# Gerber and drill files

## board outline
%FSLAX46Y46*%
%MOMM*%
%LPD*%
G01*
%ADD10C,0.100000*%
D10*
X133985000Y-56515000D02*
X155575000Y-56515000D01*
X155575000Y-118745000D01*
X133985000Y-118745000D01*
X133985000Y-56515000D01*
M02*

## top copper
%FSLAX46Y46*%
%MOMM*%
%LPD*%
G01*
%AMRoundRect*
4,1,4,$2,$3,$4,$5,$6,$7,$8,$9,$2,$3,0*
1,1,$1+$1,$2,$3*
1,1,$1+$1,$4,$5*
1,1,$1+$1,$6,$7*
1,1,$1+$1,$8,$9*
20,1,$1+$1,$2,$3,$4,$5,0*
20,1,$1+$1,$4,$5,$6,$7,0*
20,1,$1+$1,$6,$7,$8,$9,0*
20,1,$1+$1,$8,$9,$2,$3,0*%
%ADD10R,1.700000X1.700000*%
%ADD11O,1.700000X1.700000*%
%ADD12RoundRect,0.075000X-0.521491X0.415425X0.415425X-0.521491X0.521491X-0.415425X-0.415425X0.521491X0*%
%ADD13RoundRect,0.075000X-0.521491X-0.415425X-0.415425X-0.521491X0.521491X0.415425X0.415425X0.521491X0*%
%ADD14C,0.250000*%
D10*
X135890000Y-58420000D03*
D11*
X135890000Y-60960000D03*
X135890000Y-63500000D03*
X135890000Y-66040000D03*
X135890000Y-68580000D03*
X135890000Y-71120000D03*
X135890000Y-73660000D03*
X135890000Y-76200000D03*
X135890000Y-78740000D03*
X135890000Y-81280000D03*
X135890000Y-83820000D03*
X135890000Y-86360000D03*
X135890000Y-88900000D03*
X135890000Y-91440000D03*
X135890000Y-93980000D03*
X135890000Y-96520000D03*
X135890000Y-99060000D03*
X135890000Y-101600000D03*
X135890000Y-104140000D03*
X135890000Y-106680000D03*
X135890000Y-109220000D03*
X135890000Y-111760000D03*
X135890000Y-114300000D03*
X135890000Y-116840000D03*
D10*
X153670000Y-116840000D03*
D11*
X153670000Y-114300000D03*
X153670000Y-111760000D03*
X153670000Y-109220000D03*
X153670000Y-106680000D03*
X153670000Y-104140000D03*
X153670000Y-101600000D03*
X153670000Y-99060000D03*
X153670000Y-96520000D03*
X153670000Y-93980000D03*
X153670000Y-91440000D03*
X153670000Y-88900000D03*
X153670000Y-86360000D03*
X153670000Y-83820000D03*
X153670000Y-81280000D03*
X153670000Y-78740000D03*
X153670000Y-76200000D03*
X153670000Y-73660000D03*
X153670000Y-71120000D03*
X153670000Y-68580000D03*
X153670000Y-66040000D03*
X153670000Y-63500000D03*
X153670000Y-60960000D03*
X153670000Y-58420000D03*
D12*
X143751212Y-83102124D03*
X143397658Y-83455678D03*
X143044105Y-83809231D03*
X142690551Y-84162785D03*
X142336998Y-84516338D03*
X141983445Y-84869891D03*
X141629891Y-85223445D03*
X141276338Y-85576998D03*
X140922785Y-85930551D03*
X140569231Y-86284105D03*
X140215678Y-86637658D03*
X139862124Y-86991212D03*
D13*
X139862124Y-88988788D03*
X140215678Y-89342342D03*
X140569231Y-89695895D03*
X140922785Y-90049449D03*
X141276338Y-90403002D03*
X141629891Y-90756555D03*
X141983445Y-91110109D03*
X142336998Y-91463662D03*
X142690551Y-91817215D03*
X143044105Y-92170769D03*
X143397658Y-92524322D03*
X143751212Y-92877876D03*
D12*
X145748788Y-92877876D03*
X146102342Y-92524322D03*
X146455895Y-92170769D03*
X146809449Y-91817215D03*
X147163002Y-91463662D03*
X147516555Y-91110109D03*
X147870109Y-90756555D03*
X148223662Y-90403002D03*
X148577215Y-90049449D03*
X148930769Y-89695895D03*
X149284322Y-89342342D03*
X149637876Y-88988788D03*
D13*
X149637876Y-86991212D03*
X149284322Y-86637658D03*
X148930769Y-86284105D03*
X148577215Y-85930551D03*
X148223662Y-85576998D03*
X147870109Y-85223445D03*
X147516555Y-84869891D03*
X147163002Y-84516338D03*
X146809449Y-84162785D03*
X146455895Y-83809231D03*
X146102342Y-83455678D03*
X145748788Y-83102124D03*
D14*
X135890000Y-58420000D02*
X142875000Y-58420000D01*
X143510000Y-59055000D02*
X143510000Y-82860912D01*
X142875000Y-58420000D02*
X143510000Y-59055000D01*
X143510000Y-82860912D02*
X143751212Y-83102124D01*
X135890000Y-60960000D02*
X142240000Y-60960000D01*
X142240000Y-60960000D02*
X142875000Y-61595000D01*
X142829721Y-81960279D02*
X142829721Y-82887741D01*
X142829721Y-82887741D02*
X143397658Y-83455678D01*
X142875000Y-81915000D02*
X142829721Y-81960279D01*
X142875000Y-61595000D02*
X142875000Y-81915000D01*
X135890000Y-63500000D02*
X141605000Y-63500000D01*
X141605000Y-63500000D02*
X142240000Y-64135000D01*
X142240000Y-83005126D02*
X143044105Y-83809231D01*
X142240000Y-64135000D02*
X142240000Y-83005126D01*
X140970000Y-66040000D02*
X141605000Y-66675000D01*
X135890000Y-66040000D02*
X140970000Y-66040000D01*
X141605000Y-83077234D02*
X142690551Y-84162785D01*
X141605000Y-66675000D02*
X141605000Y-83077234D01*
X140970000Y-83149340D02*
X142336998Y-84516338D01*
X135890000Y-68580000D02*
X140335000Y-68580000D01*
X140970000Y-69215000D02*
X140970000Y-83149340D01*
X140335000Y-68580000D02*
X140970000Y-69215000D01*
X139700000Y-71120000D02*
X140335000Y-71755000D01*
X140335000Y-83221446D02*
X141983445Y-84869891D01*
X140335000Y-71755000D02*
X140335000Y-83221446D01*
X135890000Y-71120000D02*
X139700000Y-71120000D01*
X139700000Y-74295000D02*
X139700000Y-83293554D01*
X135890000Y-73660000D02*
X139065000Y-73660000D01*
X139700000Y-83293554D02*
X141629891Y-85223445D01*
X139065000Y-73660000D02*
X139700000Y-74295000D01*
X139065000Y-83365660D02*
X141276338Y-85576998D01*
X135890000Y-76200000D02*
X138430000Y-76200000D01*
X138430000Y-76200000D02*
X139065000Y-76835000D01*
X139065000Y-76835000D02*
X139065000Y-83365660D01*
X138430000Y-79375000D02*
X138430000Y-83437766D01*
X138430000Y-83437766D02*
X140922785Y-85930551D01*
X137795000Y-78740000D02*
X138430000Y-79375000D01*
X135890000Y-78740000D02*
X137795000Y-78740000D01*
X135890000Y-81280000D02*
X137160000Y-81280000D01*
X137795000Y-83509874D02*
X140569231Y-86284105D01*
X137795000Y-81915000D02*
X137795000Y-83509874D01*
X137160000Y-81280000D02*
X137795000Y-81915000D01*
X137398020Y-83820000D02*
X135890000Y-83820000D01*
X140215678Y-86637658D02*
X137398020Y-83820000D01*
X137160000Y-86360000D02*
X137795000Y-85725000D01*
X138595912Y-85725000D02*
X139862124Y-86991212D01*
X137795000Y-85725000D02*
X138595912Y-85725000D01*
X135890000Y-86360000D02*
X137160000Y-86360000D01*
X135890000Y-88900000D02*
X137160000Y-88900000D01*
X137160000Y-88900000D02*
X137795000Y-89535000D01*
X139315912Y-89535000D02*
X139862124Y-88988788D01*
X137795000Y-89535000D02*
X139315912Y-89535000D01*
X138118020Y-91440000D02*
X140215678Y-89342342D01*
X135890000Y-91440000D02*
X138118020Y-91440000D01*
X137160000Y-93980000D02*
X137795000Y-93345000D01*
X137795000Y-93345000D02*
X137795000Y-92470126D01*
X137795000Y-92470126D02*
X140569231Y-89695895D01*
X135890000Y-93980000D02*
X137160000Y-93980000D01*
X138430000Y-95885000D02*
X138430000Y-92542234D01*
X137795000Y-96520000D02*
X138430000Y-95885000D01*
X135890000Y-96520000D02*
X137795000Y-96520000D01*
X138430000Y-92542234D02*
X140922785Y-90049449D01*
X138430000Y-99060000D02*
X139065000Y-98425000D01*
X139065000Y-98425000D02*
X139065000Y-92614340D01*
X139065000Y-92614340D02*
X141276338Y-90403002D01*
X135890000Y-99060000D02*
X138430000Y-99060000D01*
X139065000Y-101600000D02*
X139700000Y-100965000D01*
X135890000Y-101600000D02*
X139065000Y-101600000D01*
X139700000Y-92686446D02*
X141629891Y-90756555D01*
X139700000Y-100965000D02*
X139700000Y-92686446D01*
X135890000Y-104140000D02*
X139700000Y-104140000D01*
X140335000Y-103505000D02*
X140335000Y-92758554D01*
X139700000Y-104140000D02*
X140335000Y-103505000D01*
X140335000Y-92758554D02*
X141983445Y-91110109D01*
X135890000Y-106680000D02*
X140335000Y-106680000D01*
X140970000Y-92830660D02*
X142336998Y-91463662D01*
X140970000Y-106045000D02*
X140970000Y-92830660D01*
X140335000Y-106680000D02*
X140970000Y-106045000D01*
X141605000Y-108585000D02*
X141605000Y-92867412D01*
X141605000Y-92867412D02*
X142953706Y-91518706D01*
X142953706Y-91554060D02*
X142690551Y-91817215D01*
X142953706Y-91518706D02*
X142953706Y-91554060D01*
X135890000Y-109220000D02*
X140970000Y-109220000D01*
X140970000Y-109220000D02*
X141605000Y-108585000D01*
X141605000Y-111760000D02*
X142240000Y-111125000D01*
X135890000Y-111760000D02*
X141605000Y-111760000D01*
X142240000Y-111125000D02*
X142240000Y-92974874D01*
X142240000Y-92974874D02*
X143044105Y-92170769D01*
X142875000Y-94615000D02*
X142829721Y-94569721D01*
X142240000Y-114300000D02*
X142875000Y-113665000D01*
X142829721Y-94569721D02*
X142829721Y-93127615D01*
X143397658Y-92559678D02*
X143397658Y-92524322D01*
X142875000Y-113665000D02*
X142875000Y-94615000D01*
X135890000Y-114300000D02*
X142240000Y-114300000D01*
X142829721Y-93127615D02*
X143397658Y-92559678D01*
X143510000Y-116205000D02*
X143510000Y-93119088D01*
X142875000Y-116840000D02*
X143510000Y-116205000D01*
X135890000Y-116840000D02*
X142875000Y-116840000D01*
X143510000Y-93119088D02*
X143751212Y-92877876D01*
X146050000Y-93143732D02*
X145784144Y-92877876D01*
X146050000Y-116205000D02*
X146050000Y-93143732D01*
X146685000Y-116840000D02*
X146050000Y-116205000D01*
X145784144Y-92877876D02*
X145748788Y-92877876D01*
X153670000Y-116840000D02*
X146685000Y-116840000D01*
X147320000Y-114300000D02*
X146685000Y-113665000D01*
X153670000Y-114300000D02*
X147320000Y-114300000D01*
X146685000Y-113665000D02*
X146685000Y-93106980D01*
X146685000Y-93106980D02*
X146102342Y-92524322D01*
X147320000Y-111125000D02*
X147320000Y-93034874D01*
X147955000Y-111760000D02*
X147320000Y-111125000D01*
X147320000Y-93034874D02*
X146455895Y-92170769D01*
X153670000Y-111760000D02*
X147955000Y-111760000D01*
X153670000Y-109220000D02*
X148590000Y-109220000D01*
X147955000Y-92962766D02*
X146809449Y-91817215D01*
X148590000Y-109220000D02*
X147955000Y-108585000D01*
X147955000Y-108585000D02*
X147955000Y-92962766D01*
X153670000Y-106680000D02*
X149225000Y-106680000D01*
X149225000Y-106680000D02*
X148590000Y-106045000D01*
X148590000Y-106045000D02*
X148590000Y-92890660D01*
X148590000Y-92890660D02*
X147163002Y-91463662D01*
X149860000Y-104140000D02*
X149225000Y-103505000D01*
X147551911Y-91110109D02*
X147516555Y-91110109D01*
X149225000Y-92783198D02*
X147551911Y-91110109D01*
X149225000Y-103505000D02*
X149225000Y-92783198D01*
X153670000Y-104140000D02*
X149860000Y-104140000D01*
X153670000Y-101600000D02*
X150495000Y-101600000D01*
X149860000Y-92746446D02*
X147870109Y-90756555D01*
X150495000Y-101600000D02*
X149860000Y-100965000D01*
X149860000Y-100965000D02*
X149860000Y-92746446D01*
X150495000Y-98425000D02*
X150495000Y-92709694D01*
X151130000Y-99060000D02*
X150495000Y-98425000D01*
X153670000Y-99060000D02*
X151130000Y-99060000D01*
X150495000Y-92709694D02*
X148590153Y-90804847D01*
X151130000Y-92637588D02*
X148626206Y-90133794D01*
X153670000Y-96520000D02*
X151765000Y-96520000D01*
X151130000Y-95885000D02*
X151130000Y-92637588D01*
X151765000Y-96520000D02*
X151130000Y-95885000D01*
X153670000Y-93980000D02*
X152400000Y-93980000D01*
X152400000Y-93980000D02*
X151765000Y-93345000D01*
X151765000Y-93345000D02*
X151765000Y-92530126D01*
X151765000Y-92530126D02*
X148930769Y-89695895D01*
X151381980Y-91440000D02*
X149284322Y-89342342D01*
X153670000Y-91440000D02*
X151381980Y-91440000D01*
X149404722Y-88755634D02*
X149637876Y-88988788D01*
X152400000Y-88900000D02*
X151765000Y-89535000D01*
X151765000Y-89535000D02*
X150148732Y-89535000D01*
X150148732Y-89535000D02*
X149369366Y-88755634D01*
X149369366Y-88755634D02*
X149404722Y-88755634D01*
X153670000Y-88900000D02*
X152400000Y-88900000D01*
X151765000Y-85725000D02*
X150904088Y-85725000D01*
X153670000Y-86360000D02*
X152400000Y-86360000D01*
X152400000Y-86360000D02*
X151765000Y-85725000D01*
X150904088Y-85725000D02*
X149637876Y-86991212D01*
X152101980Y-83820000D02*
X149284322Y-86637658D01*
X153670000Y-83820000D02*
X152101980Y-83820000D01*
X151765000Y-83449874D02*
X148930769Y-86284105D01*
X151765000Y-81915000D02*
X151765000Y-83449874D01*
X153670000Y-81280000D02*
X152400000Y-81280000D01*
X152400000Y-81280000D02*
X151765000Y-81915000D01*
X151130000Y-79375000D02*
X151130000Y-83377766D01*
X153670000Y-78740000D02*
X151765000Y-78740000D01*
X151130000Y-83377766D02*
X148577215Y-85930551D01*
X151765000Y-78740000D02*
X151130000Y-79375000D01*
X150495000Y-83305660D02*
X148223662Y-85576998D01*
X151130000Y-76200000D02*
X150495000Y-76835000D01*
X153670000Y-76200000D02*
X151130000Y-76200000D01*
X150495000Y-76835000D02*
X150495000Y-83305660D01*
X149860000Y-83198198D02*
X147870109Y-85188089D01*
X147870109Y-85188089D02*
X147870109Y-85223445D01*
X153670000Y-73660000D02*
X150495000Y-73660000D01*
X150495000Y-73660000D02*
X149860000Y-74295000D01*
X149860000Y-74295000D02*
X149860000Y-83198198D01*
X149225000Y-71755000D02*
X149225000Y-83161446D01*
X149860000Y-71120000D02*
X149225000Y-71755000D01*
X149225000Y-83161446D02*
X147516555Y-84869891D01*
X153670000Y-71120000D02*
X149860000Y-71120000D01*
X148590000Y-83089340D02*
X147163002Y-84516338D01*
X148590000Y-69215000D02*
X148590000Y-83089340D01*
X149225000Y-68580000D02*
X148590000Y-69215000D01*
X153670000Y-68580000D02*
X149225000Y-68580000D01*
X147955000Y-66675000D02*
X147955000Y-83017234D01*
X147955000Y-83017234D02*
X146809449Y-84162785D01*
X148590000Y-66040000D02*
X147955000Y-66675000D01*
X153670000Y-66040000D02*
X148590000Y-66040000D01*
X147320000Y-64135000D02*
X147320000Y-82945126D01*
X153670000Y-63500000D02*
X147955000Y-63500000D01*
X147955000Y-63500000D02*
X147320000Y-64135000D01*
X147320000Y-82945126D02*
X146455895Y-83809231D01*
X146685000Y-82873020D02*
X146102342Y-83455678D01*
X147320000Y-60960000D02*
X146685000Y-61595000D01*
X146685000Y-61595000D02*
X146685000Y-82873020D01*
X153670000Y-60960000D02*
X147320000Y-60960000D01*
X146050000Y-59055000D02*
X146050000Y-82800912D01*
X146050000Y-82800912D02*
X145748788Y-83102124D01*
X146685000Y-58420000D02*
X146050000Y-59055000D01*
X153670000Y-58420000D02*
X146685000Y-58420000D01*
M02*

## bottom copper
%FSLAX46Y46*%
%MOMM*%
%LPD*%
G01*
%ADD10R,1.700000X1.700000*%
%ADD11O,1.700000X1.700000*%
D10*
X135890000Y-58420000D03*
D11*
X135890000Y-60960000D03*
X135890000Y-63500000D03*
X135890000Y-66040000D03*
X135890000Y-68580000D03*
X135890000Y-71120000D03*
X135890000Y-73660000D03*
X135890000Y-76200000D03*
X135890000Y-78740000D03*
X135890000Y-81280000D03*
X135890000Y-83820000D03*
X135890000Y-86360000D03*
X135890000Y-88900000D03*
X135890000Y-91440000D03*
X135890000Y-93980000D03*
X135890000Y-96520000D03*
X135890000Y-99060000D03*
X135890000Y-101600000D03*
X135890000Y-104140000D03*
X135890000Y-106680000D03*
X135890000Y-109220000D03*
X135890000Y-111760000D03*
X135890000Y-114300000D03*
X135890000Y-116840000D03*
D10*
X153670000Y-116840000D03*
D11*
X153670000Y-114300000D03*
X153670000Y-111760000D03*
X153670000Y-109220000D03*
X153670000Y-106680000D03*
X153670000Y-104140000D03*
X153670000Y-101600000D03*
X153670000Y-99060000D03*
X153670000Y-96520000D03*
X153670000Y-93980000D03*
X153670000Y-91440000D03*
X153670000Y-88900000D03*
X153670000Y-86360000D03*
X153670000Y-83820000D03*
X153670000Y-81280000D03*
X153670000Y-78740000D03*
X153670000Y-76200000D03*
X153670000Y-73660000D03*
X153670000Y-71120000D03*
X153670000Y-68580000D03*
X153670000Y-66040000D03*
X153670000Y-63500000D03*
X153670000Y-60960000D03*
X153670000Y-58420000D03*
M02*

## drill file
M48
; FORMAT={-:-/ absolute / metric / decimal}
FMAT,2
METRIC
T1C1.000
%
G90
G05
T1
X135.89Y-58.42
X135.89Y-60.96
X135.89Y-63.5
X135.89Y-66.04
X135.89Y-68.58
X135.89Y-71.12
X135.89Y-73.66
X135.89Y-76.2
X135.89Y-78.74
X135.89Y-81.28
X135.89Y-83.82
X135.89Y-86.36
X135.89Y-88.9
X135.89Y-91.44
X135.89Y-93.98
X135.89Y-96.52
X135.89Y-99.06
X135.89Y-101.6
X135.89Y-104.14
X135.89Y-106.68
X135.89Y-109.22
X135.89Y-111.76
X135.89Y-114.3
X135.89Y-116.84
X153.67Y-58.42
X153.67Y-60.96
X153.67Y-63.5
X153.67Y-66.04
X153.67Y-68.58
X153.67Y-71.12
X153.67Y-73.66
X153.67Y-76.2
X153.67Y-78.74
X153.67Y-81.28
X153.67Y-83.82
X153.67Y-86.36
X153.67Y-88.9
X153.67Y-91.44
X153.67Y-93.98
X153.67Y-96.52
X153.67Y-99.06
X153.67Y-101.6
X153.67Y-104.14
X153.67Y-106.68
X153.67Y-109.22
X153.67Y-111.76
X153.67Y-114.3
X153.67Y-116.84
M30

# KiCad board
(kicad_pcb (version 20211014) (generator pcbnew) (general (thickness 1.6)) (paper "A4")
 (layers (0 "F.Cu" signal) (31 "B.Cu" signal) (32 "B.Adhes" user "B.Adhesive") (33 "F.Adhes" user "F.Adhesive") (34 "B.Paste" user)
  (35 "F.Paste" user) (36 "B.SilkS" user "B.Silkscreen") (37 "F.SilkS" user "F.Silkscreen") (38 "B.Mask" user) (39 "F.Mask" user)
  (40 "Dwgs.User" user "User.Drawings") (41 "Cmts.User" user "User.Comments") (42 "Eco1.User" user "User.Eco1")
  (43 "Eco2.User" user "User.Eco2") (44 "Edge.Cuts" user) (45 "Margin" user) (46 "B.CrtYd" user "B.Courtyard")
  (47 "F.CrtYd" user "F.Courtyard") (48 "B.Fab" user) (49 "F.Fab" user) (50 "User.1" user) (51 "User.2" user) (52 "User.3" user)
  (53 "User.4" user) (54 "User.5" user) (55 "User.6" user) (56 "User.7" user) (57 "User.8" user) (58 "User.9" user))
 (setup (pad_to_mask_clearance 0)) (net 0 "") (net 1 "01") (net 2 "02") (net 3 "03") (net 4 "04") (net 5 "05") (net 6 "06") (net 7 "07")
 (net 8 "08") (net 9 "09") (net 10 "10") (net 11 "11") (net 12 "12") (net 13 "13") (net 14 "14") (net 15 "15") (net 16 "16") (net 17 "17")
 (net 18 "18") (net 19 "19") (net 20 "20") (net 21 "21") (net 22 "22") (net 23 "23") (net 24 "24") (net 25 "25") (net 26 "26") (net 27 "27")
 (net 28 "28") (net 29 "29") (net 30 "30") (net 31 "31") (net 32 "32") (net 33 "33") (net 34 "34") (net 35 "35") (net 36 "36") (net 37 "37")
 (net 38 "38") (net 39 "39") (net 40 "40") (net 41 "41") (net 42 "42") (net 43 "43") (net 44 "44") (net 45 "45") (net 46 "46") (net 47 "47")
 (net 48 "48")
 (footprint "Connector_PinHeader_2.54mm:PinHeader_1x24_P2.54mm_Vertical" (layer "F.Cu") (at 135.89 58.42)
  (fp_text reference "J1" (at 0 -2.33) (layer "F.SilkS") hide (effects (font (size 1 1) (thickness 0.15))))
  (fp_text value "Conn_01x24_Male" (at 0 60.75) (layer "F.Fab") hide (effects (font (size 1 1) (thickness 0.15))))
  (pad "1" thru_hole rect (at 0 0) (size 1.7 1.7) (drill 1) (layers *.Cu *.Mask) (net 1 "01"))
  (pad "2" thru_hole oval (at 0 2.54) (size 1.7 1.7) (drill 1) (layers *.Cu *.Mask) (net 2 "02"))
  (pad "3" thru_hole oval (at 0 5.08) (size 1.7 1.7) (drill 1) (layers *.Cu *.Mask) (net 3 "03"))
  (pad "4" thru_hole oval (at 0 7.62) (size 1.7 1.7) (drill 1) (layers *.Cu *.Mask) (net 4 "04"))
  (pad "5" thru_hole oval (at 0 10.16) (size 1.7 1.7) (drill 1) (layers *.Cu *.Mask) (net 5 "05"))
  (pad "6" thru_hole oval (at 0 12.7) (size 1.7 1.7) (drill 1) (layers *.Cu *.Mask) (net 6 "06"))
  (pad "7" thru_hole oval (at 0 15.24) (size 1.7 1.7) (drill 1) (layers *.Cu *.Mask) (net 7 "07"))
  (pad "8" thru_hole oval (at 0 17.78) (size 1.7 1.7) (drill 1) (layers *.Cu *.Mask) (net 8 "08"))
  (pad "9" thru_hole oval (at 0 20.32) (size 1.7 1.7) (drill 1) (layers *.Cu *.Mask) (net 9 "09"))
  (pad "10" thru_hole oval (at 0 22.86) (size 1.7 1.7) (drill 1) (layers *.Cu *.Mask) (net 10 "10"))
  (pad "11" thru_hole oval (at 0 25.4) (size 1.7 1.7) (drill 1) (layers *.Cu *.Mask) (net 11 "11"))
  (pad "12" thru_hole oval (at 0 27.94) (size 1.7 1.7) (drill 1) (layers *.Cu *.Mask) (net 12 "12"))
  (pad "13" thru_hole oval (at 0 30.48) (size 1.7 1.7) (drill 1) (layers *.Cu *.Mask) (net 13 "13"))
  (pad "14" thru_hole oval (at 0 33.02) (size 1.7 1.7) (drill 1) (layers *.Cu *.Mask) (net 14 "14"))
  (pad "15" thru_hole oval (at 0 35.56) (size 1.7 1.7) (drill 1) (layers *.Cu *.Mask) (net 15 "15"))
  (pad "16" thru_hole oval (at 0 38.1) (size 1.7 1.7) (drill 1) (layers *.Cu *.Mask) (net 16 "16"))
  (pad "17" thru_hole oval (at 0 40.64) (size 1.7 1.7) (drill 1) (layers *.Cu *.Mask) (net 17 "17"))
  (pad "18" thru_hole oval (at 0 43.18) (size 1.7 1.7) (drill 1) (layers *.Cu *.Mask) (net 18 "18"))
  (pad "19" thru_hole oval (at 0 45.72) (size 1.7 1.7) (drill 1) (layers *.Cu *.Mask) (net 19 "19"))
  (pad "20" thru_hole oval (at 0 48.26) (size 1.7 1.7) (drill 1) (layers *.Cu *.Mask) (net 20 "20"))
  (pad "21" thru_hole oval (at 0 50.8) (size 1.7 1.7) (drill 1) (layers *.Cu *.Mask) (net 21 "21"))
  (pad "22" thru_hole oval (at 0 53.34) (size 1.7 1.7) (drill 1) (layers *.Cu *.Mask) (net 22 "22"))
  (pad "23" thru_hole oval (at 0 55.88) (size 1.7 1.7) (drill 1) (layers *.Cu *.Mask) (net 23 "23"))
  (pad "24" thru_hole oval (at 0 58.42) (size 1.7 1.7) (drill 1) (layers *.Cu *.Mask) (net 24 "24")))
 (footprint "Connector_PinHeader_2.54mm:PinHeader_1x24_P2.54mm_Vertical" (layer "F.Cu") (at 153.67 116.84 180)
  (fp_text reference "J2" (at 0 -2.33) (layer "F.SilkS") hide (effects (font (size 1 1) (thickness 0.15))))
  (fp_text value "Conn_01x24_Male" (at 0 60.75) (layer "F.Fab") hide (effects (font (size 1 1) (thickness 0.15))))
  (pad "1" thru_hole rect (at 0 0 180) (size 1.7 1.7) (drill 1) (layers *.Cu *.Mask) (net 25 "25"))
  (pad "2" thru_hole oval (at 0 2.54 180) (size 1.7 1.7) (drill 1) (layers *.Cu *.Mask) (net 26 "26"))
  (pad "3" thru_hole oval (at 0 5.08 180) (size 1.7 1.7) (drill 1) (layers *.Cu *.Mask) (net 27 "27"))
  (pad "4" thru_hole oval (at 0 7.62 180) (size 1.7 1.7) (drill 1) (layers *.Cu *.Mask) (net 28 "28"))
  (pad "5" thru_hole oval (at 0 10.16 180) (size 1.7 1.7) (drill 1) (layers *.Cu *.Mask) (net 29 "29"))
  (pad "6" thru_hole oval (at 0 12.7 180) (size 1.7 1.7) (drill 1) (layers *.Cu *.Mask) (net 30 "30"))
  (pad "7" thru_hole oval (at 0 15.24 180) (size 1.7 1.7) (drill 1) (layers *.Cu *.Mask) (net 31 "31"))
  (pad "8" thru_hole oval (at 0 17.78 180) (size 1.7 1.7) (drill 1) (layers *.Cu *.Mask) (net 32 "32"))
  (pad "9" thru_hole oval (at 0 20.32 180) (size 1.7 1.7) (drill 1) (layers *.Cu *.Mask) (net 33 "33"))
  (pad "10" thru_hole oval (at 0 22.86 180) (size 1.7 1.7) (drill 1) (layers *.Cu *.Mask) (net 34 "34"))
  (pad "11" thru_hole oval (at 0 25.4 180) (size 1.7 1.7) (drill 1) (layers *.Cu *.Mask) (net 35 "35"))
  (pad "12" thru_hole oval (at 0 27.94 180) (size 1.7 1.7) (drill 1) (layers *.Cu *.Mask) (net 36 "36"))
  (pad "13" thru_hole oval (at 0 30.48 180) (size 1.7 1.7) (drill 1) (layers *.Cu *.Mask) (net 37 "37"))
  (pad "14" thru_hole oval (at 0 33.02 180) (size 1.7 1.7) (drill 1) (layers *.Cu *.Mask) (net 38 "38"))
  (pad "15" thru_hole oval (at 0 35.56 180) (size 1.7 1.7) (drill 1) (layers *.Cu *.Mask) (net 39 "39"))
  (pad "16" thru_hole oval (at 0 38.1 180) (size 1.7 1.7) (drill 1) (layers *.Cu *.Mask) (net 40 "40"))
  (pad "17" thru_hole oval (at 0 40.64 180) (size 1.7 1.7) (drill 1) (layers *.Cu *.Mask) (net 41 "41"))
  (pad "18" thru_hole oval (at 0 43.18 180) (size 1.7 1.7) (drill 1) (layers *.Cu *.Mask) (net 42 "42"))
  (pad "19" thru_hole oval (at 0 45.72 180) (size 1.7 1.7) (drill 1) (layers *.Cu *.Mask) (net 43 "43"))
  (pad "20" thru_hole oval (at 0 48.26 180) (size 1.7 1.7) (drill 1) (layers *.Cu *.Mask) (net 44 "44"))
  (pad "21" thru_hole oval (at 0 50.8 180) (size 1.7 1.7) (drill 1) (layers *.Cu *.Mask) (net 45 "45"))
  (pad "22" thru_hole oval (at 0 53.34 180) (size 1.7 1.7) (drill 1) (layers *.Cu *.Mask) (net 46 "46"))
  (pad "23" thru_hole oval (at 0 55.88 180) (size 1.7 1.7) (drill 1) (layers *.Cu *.Mask) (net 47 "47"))
  (pad "24" thru_hole oval (at 0 58.42 180) (size 1.7 1.7) (drill 1) (layers *.Cu *.Mask) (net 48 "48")))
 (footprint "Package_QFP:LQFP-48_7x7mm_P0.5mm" (layer "F.Cu") (at 144.75 87.99 -45)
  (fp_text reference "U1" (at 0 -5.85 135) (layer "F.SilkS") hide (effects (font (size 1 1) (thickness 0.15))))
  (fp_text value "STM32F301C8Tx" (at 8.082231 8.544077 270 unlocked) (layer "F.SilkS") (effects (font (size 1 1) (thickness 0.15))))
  (pad "1" smd roundrect (at -4.1625 -2.75 315) (size 1.475 0.3) (layers "F.Cu" "F.Paste" "F.Mask") (roundrect_rratio 0.25) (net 1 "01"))
  (pad "2" smd roundrect (at -4.1625 -2.25 315) (size 1.475 0.3) (layers "F.Cu" "F.Paste" "F.Mask") (roundrect_rratio 0.25) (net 2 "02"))
  (pad "3" smd roundrect (at -4.1625 -1.75 315) (size 1.475 0.3) (layers "F.Cu" "F.Paste" "F.Mask") (roundrect_rratio 0.25) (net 3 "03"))
  (pad "4" smd roundrect (at -4.1625 -1.25 315) (size 1.475 0.3) (layers "F.Cu" "F.Paste" "F.Mask") (roundrect_rratio 0.25) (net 4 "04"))
  (pad "5" smd roundrect (at -4.1625 -0.75 315) (size 1.475 0.3) (layers "F.Cu" "F.Paste" "F.Mask") (roundrect_rratio 0.25) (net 5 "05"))
  (pad "6" smd roundrect (at -4.1625 -0.25 315) (size 1.475 0.3) (layers "F.Cu" "F.Paste" "F.Mask") (roundrect_rratio 0.25) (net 6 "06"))
  (pad "7" smd roundrect (at -4.1625 0.25 315) (size 1.475 0.3) (layers "F.Cu" "F.Paste" "F.Mask") (roundrect_rratio 0.25) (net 7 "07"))
  (pad "8" smd roundrect (at -4.1625 0.75 315) (size 1.475 0.3) (layers "F.Cu" "F.Paste" "F.Mask") (roundrect_rratio 0.25) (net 8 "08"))
  (pad "9" smd roundrect (at -4.1625 1.25 315) (size 1.475 0.3) (layers "F.Cu" "F.Paste" "F.Mask") (roundrect_rratio 0.25) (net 9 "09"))
  (pad "10" smd roundrect (at -4.1625 1.75 315) (size 1.475 0.3) (layers "F.Cu" "F.Paste" "F.Mask") (roundrect_rratio 0.25) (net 10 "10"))
  (pad "11" smd roundrect (at -4.1625 2.25 315) (size 1.475 0.3) (layers "F.Cu" "F.Paste" "F.Mask") (roundrect_rratio 0.25) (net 11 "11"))
  (pad "12" smd roundrect (at -4.1625 2.75 315) (size 1.475 0.3) (layers "F.Cu" "F.Paste" "F.Mask") (roundrect_rratio 0.25) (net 12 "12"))
  (pad "13" smd roundrect (at -2.75 4.1625 315) (size 0.3 1.475) (layers "F.Cu" "F.Paste" "F.Mask") (roundrect_rratio 0.25) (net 13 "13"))
  (pad "14" smd roundrect (at -2.25 4.1625 315) (size 0.3 1.475) (layers "F.Cu" "F.Paste" "F.Mask") (roundrect_rratio 0.25) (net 14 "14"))
  (pad "15" smd roundrect (at -1.75 4.1625 315) (size 0.3 1.475) (layers "F.Cu" "F.Paste" "F.Mask") (roundrect_rratio 0.25) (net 15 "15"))
  (pad "16" smd roundrect (at -1.25 4.1625 315) (size 0.3 1.475) (layers "F.Cu" "F.Paste" "F.Mask") (roundrect_rratio 0.25) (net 16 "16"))
  (pad "17" smd roundrect (at -0.75 4.1625 315) (size 0.3 1.475) (layers "F.Cu" "F.Paste" "F.Mask") (roundrect_rratio 0.25) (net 17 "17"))
  (pad "18" smd roundrect (at -0.25 4.1625 315) (size 0.3 1.475) (layers "F.Cu" "F.Paste" "F.Mask") (roundrect_rratio 0.25) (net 18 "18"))
  (pad "19" smd roundrect (at 0.25 4.1625 315) (size 0.3 1.475) (layers "F.Cu" "F.Paste" "F.Mask") (roundrect_rratio 0.25) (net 19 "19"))
  (pad "20" smd roundrect (at 0.75 4.1625 315) (size 0.3 1.475) (layers "F.Cu" "F.Paste" "F.Mask") (roundrect_rratio 0.25) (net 20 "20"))
  (pad "21" smd roundrect (at 1.25 4.1625 315) (size 0.3 1.475) (layers "F.Cu" "F.Paste" "F.Mask") (roundrect_rratio 0.25) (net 21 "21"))
  (pad "22" smd roundrect (at 1.75 4.1625 315) (size 0.3 1.475) (layers "F.Cu" "F.Paste" "F.Mask") (roundrect_rratio 0.25) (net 22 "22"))
  (pad "23" smd roundrect (at 2.25 4.1625 315) (size 0.3 1.475) (layers "F.Cu" "F.Paste" "F.Mask") (roundrect_rratio 0.25) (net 23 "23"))
  (pad "24" smd roundrect (at 2.75 4.1625 315) (size 0.3 1.475) (layers "F.Cu" "F.Paste" "F.Mask") (roundrect_rratio 0.25) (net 24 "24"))
  (pad "25" smd roundrect (at 4.1625 2.75 315) (size 1.475 0.3) (layers "F.Cu" "F.Paste" "F.Mask") (roundrect_rratio 0.25) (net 25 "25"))
  (pad "26" smd roundrect (at 4.1625 2.25 315) (size 1.475 0.3) (layers "F.Cu" "F.Paste" "F.Mask") (roundrect_rratio 0.25) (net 26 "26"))
  (pad "27" smd roundrect (at 4.1625 1.75 315) (size 1.475 0.3) (layers "F.Cu" "F.Paste" "F.Mask") (roundrect_rratio 0.25) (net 27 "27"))
  (pad "28" smd roundrect (at 4.1625 1.25 315) (size 1.475 0.3) (layers "F.Cu" "F.Paste" "F.Mask") (roundrect_rratio 0.25) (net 28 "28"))
  (pad "29" smd roundrect (at 4.1625 0.75 315) (size 1.475 0.3) (layers "F.Cu" "F.Paste" "F.Mask") (roundrect_rratio 0.25) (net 29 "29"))
  (pad "30" smd roundrect (at 4.1625 0.25 315) (size 1.475 0.3) (layers "F.Cu" "F.Paste" "F.Mask") (roundrect_rratio 0.25) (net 30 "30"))
  (pad "31" smd roundrect (at 4.1625 -0.25 315) (size 1.475 0.3) (layers "F.Cu" "F.Paste" "F.Mask") (roundrect_rratio 0.25) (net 31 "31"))
  (pad "32" smd roundrect (at 4.1625 -0.75 315) (size 1.475 0.3) (layers "F.Cu" "F.Paste" "F.Mask") (roundrect_rratio 0.25) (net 32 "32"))
  (pad "33" smd roundrect (at 4.1625 -1.25 315) (size 1.475 0.3) (layers "F.Cu" "F.Paste" "F.Mask") (roundrect_rratio 0.25) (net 33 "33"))
  (pad "34" smd roundrect (at 4.1625 -1.75 315) (size 1.475 0.3) (layers "F.Cu" "F.Paste" "F.Mask") (roundrect_rratio 0.25) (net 34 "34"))
  (pad "35" smd roundrect (at 4.1625 -2.25 315) (size 1.475 0.3) (layers "F.Cu" "F.Paste" "F.Mask") (roundrect_rratio 0.25) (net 35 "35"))
  (pad "36" smd roundrect (at 4.1625 -2.75 315) (size 1.475 0.3) (layers "F.Cu" "F.Paste" "F.Mask") (roundrect_rratio 0.25) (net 36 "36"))
  (pad "37" smd roundrect (at 2.75 -4.1625 315) (size 0.3 1.475) (layers "F.Cu" "F.Paste" "F.Mask") (roundrect_rratio 0.25) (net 37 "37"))
  (pad "38" smd roundrect (at 2.25 -4.1625 315) (size 0.3 1.475) (layers "F.Cu" "F.Paste" "F.Mask") (roundrect_rratio 0.25) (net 38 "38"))
  (pad "39" smd roundrect (at 1.75 -4.1625 315) (size 0.3 1.475) (layers "F.Cu" "F.Paste" "F.Mask") (roundrect_rratio 0.25) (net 39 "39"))
  (pad "40" smd roundrect (at 1.25 -4.1625 315) (size 0.3 1.475) (layers "F.Cu" "F.Paste" "F.Mask") (roundrect_rratio 0.25) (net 40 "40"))
  (pad "41" smd roundrect (at 0.75 -4.1625 315) (size 0.3 1.475) (layers "F.Cu" "F.Paste" "F.Mask") (roundrect_rratio 0.25) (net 41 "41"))
  (pad "42" smd roundrect (at 0.25 -4.1625 315) (size 0.3 1.475) (layers "F.Cu" "F.Paste" "F.Mask") (roundrect_rratio 0.25) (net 42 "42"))
  (pad "43" smd roundrect (at -0.25 -4.1625 315) (size 0.3 1.475) (layers "F.Cu" "F.Paste" "F.Mask") (roundrect_rratio 0.25) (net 43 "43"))
  (pad "44" smd roundrect (at -0.75 -4.1625 315) (size 0.3 1.475) (layers "F.Cu" "F.Paste" "F.Mask") (roundrect_rratio 0.25) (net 44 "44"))
  (pad "45" smd roundrect (at -1.25 -4.1625 315) (size 0.3 1.475) (layers "F.Cu" "F.Paste" "F.Mask") (roundrect_rratio 0.25) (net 45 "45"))
  (pad "46" smd roundrect (at -1.75 -4.1625 315) (size 0.3 1.475) (layers "F.Cu" "F.Paste" "F.Mask") (roundrect_rratio 0.25) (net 46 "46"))
  (pad "47" smd roundrect (at -2.25 -4.1625 315) (size 0.3 1.475) (layers "F.Cu" "F.Paste" "F.Mask") (roundrect_rratio 0.25) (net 47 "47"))
  (pad "48" smd roundrect (at -2.75 -4.1625 315) (size 0.3 1.475) (layers "F.Cu" "F.Paste" "F.Mask") (roundrect_rratio 0.25) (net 48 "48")))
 (gr_rect (start 133.985 56.515) (end 155.575 118.745) (layer "Edge.Cuts") (width 0.1) (fill none))
 (segment (start 135.89 58.42) (end 142.875 58.42) (width 0.25) (layer "F.Cu") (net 1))
 (segment (start 143.51 59.055) (end 143.51 82.860912) (width 0.25) (layer "F.Cu") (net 1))
 (segment (start 142.875 58.42) (end 143.51 59.055) (width 0.25) (layer "F.Cu") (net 1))
 (segment (start 143.51 82.860912) (end 143.751212 83.102124) (width 0.25) (layer "F.Cu") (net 1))
 (segment (start 135.89 60.96) (end 142.24 60.96) (width 0.25) (layer "F.Cu") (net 2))
 (segment (start 142.24 60.96) (end 142.875 61.595) (width 0.25) (layer "F.Cu") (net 2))
 (segment (start 142.829721 81.960279) (end 142.829721 82.887741) (width 0.25) (layer "F.Cu") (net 2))
 (segment (start 142.829721 82.887741) (end 143.397658 83.455678) (width 0.25) (layer "F.Cu") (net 2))
 (segment (start 142.875 81.915) (end 142.829721 81.960279) (width 0.25) (layer "F.Cu") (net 2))
 (segment (start 142.875 61.595) (end 142.875 81.915) (width 0.25) (layer "F.Cu") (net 2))
 (segment (start 135.89 63.5) (end 141.605 63.5) (width 0.25) (layer "F.Cu") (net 3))
 (segment (start 141.605 63.5) (end 142.24 64.135) (width 0.25) (layer "F.Cu") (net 3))
 (segment (start 142.24 83.005126) (end 143.044105 83.809231) (width 0.25) (layer "F.Cu") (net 3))
 (segment (start 142.24 64.135) (end 142.24 83.005126) (width 0.25) (layer "F.Cu") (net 3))
 (segment (start 140.97 66.04) (end 141.605 66.675) (width 0.25) (layer "F.Cu") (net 4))
 (segment (start 135.89 66.04) (end 140.97 66.04) (width 0.25) (layer "F.Cu") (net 4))
 (segment (start 141.605 83.077234) (end 142.690551 84.162785) (width 0.25) (layer "F.Cu") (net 4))
 (segment (start 141.605 66.675) (end 141.605 83.077234) (width 0.25) (layer "F.Cu") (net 4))
 (segment (start 140.97 83.14934) (end 142.336998 84.516338) (width 0.25) (layer "F.Cu") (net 5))
 (segment (start 135.89 68.58) (end 140.335 68.58) (width 0.25) (layer "F.Cu") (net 5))
 (segment (start 140.97 69.215) (end 140.97 83.14934) (width 0.25) (layer "F.Cu") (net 5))
 (segment (start 140.335 68.58) (end 140.97 69.215) (width 0.25) (layer "F.Cu") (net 5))
 (segment (start 139.7 71.12) (end 140.335 71.755) (width 0.25) (layer "F.Cu") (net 6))
 (segment (start 140.335 83.221446) (end 141.983445 84.869891) (width 0.25) (layer "F.Cu") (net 6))
 (segment (start 140.335 71.755) (end 140.335 83.221446) (width 0.25) (layer "F.Cu") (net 6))
 (segment (start 135.89 71.12) (end 139.7 71.12) (width 0.25) (layer "F.Cu") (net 6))
 (segment (start 139.7 74.295) (end 139.7 83.293554) (width 0.25) (layer "F.Cu") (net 7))
 (segment (start 135.89 73.66) (end 139.065 73.66) (width 0.25) (layer "F.Cu") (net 7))
 (segment (start 139.7 83.293554) (end 141.629891 85.223445) (width 0.25) (layer "F.Cu") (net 7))
 (segment (start 139.065 73.66) (end 139.7 74.295) (width 0.25) (layer "F.Cu") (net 7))
 (segment (start 139.065 83.36566) (end 141.276338 85.576998) (width 0.25) (layer "F.Cu") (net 8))
 (segment (start 135.89 76.2) (end 138.43 76.2) (width 0.25) (layer "F.Cu") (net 8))
 (segment (start 138.43 76.2) (end 139.065 76.835) (width 0.25) (layer "F.Cu") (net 8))
 (segment (start 139.065 76.835) (end 139.065 83.36566) (width 0.25) (layer "F.Cu") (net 8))
 (segment (start 138.43 79.375) (end 138.43 83.437766) (width 0.25) (layer "F.Cu") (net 9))
 (segment (start 138.43 83.437766) (end 140.922785 85.930551) (width 0.25) (layer "F.Cu") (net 9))
 (segment (start 137.795 78.74) (end 138.43 79.375) (width 0.25) (layer "F.Cu") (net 9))
 (segment (start 135.89 78.74) (end 137.795 78.74) (width 0.25) (layer "F.Cu") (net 9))
 (segment (start 135.89 81.28) (end 137.16 81.28) (width 0.25) (layer "F.Cu") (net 10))
 (segment (start 137.795 83.509874) (end 140.569231 86.284105) (width 0.25) (layer "F.Cu") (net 10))
 (segment (start 137.795 81.915) (end 137.795 83.509874) (width 0.25) (layer "F.Cu") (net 10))
 (segment (start 137.16 81.28) (end 137.795 81.915) (width 0.25) (layer "F.Cu") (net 10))
 (segment (start 137.39802 83.82) (end 135.89 83.82) (width 0.25) (layer "F.Cu") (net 11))
 (segment (start 140.215678 86.637658) (end 137.39802 83.82) (width 0.25) (layer "F.Cu") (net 11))
 (segment (start 137.16 86.36) (end 137.795 85.725) (width 0.25) (layer "F.Cu") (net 12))
 (segment (start 138.595912 85.725) (end 139.862124 86.991212) (width 0.25) (layer "F.Cu") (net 12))
 (segment (start 137.795 85.725) (end 138.595912 85.725) (width 0.25) (layer "F.Cu") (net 12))
 (segment (start 135.89 86.36) (end 137.16 86.36) (width 0.25) (layer "F.Cu") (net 12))
 (segment (start 135.89 88.9) (end 137.16 88.9) (width 0.25) (layer "F.Cu") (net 13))
 (segment (start 137.16 88.9) (end 137.795 89.535) (width 0.25) (layer "F.Cu") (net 13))
 (segment (start 139.315912 89.535) (end 139.862124 88.988788) (width 0.25) (layer "F.Cu") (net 13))
 (segment (start 137.795 89.535) (end 139.315912 89.535) (width 0.25) (layer "F.Cu") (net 13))
 (segment (start 138.11802 91.44) (end 140.215678 89.342342) (width 0.25) (layer "F.Cu") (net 14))
 (segment (start 135.89 91.44) (end 138.11802 91.44) (width 0.25) (layer "F.Cu") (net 14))
 (segment (start 137.16 93.98) (end 137.795 93.345) (width 0.25) (layer "F.Cu") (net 15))
 (segment (start 137.795 93.345) (end 137.795 92.470126) (width 0.25) (layer "F.Cu") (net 15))
 (segment (start 137.795 92.470126) (end 140.569231 89.695895) (width 0.25) (layer "F.Cu") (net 15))
 (segment (start 135.89 93.98) (end 137.16 93.98) (width 0.25) (layer "F.Cu") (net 15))
 (segment (start 138.43 95.885) (end 138.43 92.542234) (width 0.25) (layer "F.Cu") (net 16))
 (segment (start 137.795 96.52) (end 138.43 95.885) (width 0.25) (layer "F.Cu") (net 16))
 (segment (start 135.89 96.52) (end 137.795 96.52) (width 0.25) (layer "F.Cu") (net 16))
 (segment (start 138.43 92.542234) (end 140.922785 90.049449) (width 0.25) (layer "F.Cu") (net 16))
 (segment (start 138.43 99.06) (end 139.065 98.425) (width 0.25) (layer "F.Cu") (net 17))
 (segment (start 139.065 98.425) (end 139.065 92.61434) (width 0.25) (layer "F.Cu") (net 17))
 (segment (start 139.065 92.61434) (end 141.276338 90.403002) (width 0.25) (layer "F.Cu") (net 17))
 (segment (start 135.89 99.06) (end 138.43 99.06) (width 0.25) (layer "F.Cu") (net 17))
 (segment (start 139.065 101.6) (end 139.7 100.965) (width 0.25) (layer "F.Cu") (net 18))
 (segment (start 135.89 101.6) (end 139.065 101.6) (width 0.25) (layer "F.Cu") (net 18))
 (segment (start 139.7 92.686446) (end 141.629891 90.756555) (width 0.25) (layer "F.Cu") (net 18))
 (segment (start 139.7 100.965) (end 139.7 92.686446) (width 0.25) (layer "F.Cu") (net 18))
 (segment (start 135.89 104.14) (end 139.7 104.14) (width 0.25) (layer "F.Cu") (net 19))
 (segment (start 140.335 103.505) (end 140.335 92.758554) (width 0.25) (layer "F.Cu") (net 19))
 (segment (start 139.7 104.14) (end 140.335 103.505) (width 0.25) (layer "F.Cu") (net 19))
 (segment (start 140.335 92.758554) (end 141.983445 91.110109) (width 0.25) (layer "F.Cu") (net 19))
 (segment (start 135.89 106.68) (end 140.335 106.68) (width 0.25) (layer "F.Cu") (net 20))
 (segment (start 140.97 92.83066) (end 142.336998 91.463662) (width 0.25) (layer "F.Cu") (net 20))
 (segment (start 140.97 106.045) (end 140.97 92.83066) (width 0.25) (layer "F.Cu") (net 20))
 (segment (start 140.335 106.68) (end 140.97 106.045) (width 0.25) (layer "F.Cu") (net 20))
 (segment (start 141.605 108.585) (end 141.605 92.867412) (width 0.25) (layer "F.Cu") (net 21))
 (segment (start 141.605 92.867412) (end 142.953706 91.518706) (width 0.25) (layer "F.Cu") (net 21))
 (segment (start 142.953706 91.55406) (end 142.690551 91.817215) (width 0.25) (layer "F.Cu") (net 21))
 (segment (start 142.953706 91.518706) (end 142.953706 91.55406) (width 0.25) (layer "F.Cu") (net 21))
 (segment (start 135.89 109.22) (end 140.97 109.22) (width 0.25) (layer "F.Cu") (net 21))
 (segment (start 140.97 109.22) (end 141.605 108.585) (width 0.25) (layer "F.Cu") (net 21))
 (segment (start 141.605 111.76) (end 142.24 111.125) (width 0.25) (layer "F.Cu") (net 22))
 (segment (start 135.89 111.76) (end 141.605 111.76) (width 0.25) (layer "F.Cu") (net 22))
 (segment (start 142.24 111.125) (end 142.24 92.974874) (width 0.25) (layer "F.Cu") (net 22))
 (segment (start 142.24 92.974874) (end 143.044105 92.170769) (width 0.25) (layer "F.Cu") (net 22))
 (segment (start 142.875 94.615) (end 142.829721 94.569721) (width 0.25) (layer "F.Cu") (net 23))
 (segment (start 142.24 114.3) (end 142.875 113.665) (width 0.25) (layer "F.Cu") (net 23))
 (segment (start 142.829721 94.569721) (end 142.829721 93.127615) (width 0.25) (layer "F.Cu") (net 23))
 (segment (start 143.397658 92.559678) (end 143.397658 92.524322) (width 0.25) (layer "F.Cu") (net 23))
 (segment (start 142.875 113.665) (end 142.875 94.615) (width 0.25) (layer "F.Cu") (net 23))
 (segment (start 135.89 114.3) (end 142.24 114.3) (width 0.25) (layer "F.Cu") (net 23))
 (segment (start 142.829721 93.127615) (end 143.397658 92.559678) (width 0.25) (layer "F.Cu") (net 23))
 (segment (start 143.51 116.205) (end 143.51 93.119088) (width 0.25) (layer "F.Cu") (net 24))
 (segment (start 142.875 116.84) (end 143.51 116.205) (width 0.25) (layer "F.Cu") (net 24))
 (segment (start 135.89 116.84) (end 142.875 116.84) (width 0.25) (layer "F.Cu") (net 24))
 (segment (start 143.51 93.119088) (end 143.751212 92.877876) (width 0.25) (layer "F.Cu") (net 24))
 (segment (start 146.05 93.143732) (end 145.784144 92.877876) (width 0.25) (layer "F.Cu") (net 25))
 (segment (start 146.05 116.205) (end 146.05 93.143732) (width 0.25) (layer "F.Cu") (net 25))
 (segment (start 146.685 116.84) (end 146.05 116.205) (width 0.25) (layer "F.Cu") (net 25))
 (segment (start 145.784144 92.877876) (end 145.748788 92.877876) (width 0.25) (layer "F.Cu") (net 25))
 (segment (start 153.67 116.84) (end 146.685 116.84) (width 0.25) (layer "F.Cu") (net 25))
 (segment (start 147.32 114.3) (end 146.685 113.665) (width 0.25) (layer "F.Cu") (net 26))
 (segment (start 153.67 114.3) (end 147.32 114.3) (width 0.25) (layer "F.Cu") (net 26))
 (segment (start 146.685 113.665) (end 146.685 93.10698) (width 0.25) (layer "F.Cu") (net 26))
 (segment (start 146.685 93.10698) (end 146.102342 92.524322) (width 0.25) (layer "F.Cu") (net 26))
 (segment (start 147.32 111.125) (end 147.32 93.034874) (width 0.25) (layer "F.Cu") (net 27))
 (segment (start 147.955 111.76) (end 147.32 111.125) (width 0.25) (layer "F.Cu") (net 27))
 (segment (start 147.32 93.034874) (end 146.455895 92.170769) (width 0.25) (layer "F.Cu") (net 27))
 (segment (start 153.67 111.76) (end 147.955 111.76) (width 0.25) (layer "F.Cu") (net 27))
 (segment (start 153.67 109.22) (end 148.59 109.22) (width 0.25) (layer "F.Cu") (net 28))
 (segment (start 147.955 92.962766) (end 146.809449 91.817215) (width 0.25) (layer "F.Cu") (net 28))
 (segment (start 148.59 109.22) (end 147.955 108.585) (width 0.25) (layer "F.Cu") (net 28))
 (segment (start 147.955 108.585) (end 147.955 92.962766) (width 0.25) (layer "F.Cu") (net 28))
 (segment (start 153.67 106.68) (end 149.225 106.68) (width 0.25) (layer "F.Cu") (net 29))
 (segment (start 149.225 106.68) (end 148.59 106.045) (width 0.25) (layer "F.Cu") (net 29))
 (segment (start 148.59 106.045) (end 148.59 92.89066) (width 0.25) (layer "F.Cu") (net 29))
 (segment (start 148.59 92.89066) (end 147.163002 91.463662) (width 0.25) (layer "F.Cu") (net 29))
 (segment (start 149.86 104.14) (end 149.225 103.505) (width 0.25) (layer "F.Cu") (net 30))
 (segment (start 147.551911 91.110109) (end 147.516555 91.110109) (width 0.25) (layer "F.Cu") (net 30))
 (segment (start 149.225 92.783198) (end 147.551911 91.110109) (width 0.25) (layer "F.Cu") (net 30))
 (segment (start 149.225 103.505) (end 149.225 92.783198) (width 0.25) (layer "F.Cu") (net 30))
 (segment (start 153.67 104.14) (end 149.86 104.14) (width 0.25) (layer "F.Cu") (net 30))
 (segment (start 153.67 101.6) (end 150.495 101.6) (width 0.25) (layer "F.Cu") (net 31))
 (segment (start 149.86 92.746446) (end 147.870109 90.756555) (width 0.25) (layer "F.Cu") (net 31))
 (segment (start 150.495 101.6) (end 149.86 100.965) (width 0.25) (layer "F.Cu") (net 31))
 (segment (start 149.86 100.965) (end 149.86 92.746446) (width 0.25) (layer "F.Cu") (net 31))
 (segment (start 150.495 98.425) (end 150.495 92.709694) (width 0.25) (layer "F.Cu") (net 32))
 (segment (start 151.13 99.06) (end 150.495 98.425) (width 0.25) (layer "F.Cu") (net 32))
 (segment (start 153.67 99.06) (end 151.13 99.06) (width 0.25) (layer "F.Cu") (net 32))
 (segment (start 150.495 92.709694) (end 148.590153 90.804847) (width 0.25) (layer "F.Cu") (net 32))
 (segment (start 151.13 92.637588) (end 148.626206 90.133794) (width 0.25) (layer "F.Cu") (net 33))
 (segment (start 153.67 96.52) (end 151.765 96.52) (width 0.25) (layer "F.Cu") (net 33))
 (segment (start 151.13 95.885) (end 151.13 92.637588) (width 0.25) (layer "F.Cu") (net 33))
 (segment (start 151.765 96.52) (end 151.13 95.885) (width 0.25) (layer "F.Cu") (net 33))
 (segment (start 153.67 93.98) (end 152.4 93.98) (width 0.25) (layer "F.Cu") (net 34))
 (segment (start 152.4 93.98) (end 151.765 93.345) (width 0.25) (layer "F.Cu") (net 34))
 (segment (start 151.765 93.345) (end 151.765 92.530126) (width 0.25) (layer "F.Cu") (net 34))
 (segment (start 151.765 92.530126) (end 148.930769 89.695895) (width 0.25) (layer "F.Cu") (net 34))
 (segment (start 151.38198 91.44) (end 149.284322 89.342342) (width 0.25) (layer "F.Cu") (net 35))
 (segment (start 153.67 91.44) (end 151.38198 91.44) (width 0.25) (layer "F.Cu") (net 35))
 (segment (start 149.404722 88.755634) (end 149.637876 88.988788) (width 0.25) (layer "F.Cu") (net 36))
 (segment (start 152.4 88.9) (end 151.765 89.535) (width 0.25) (layer "F.Cu") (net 36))
 (segment (start 151.765 89.535) (end 150.148732 89.535) (width 0.25) (layer "F.Cu") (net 36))
 (segment (start 150.148732 89.535) (end 149.369366 88.755634) (width 0.25) (layer "F.Cu") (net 36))
 (segment (start 149.369366 88.755634) (end 149.404722 88.755634) (width 0.25) (layer "F.Cu") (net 36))
 (segment (start 153.67 88.9) (end 152.4 88.9) (width 0.25) (layer "F.Cu") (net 36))
 (segment (start 151.765 85.725) (end 150.904088 85.725) (width 0.25) (layer "F.Cu") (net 37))
 (segment (start 153.67 86.36) (end 152.4 86.36) (width 0.25) (layer "F.Cu") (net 37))
 (segment (start 152.4 86.36) (end 151.765 85.725) (width 0.25) (layer "F.Cu") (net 37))
 (segment (start 150.904088 85.725) (end 149.637876 86.991212) (width 0.25) (layer "F.Cu") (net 37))
 (segment (start 152.10198 83.82) (end 149.284322 86.637658) (width 0.25) (layer "F.Cu") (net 38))
 (segment (start 153.67 83.82) (end 152.10198 83.82) (width 0.25) (layer "F.Cu") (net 38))
 (segment (start 151.765 83.449874) (end 148.930769 86.284105) (width 0.25) (layer "F.Cu") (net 39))
 (segment (start 151.765 81.915) (end 151.765 83.449874) (width 0.25) (layer "F.Cu") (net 39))
 (segment (start 153.67 81.28) (end 152.4 81.28) (width 0.25) (layer "F.Cu") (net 39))
 (segment (start 152.4 81.28) (end 151.765 81.915) (width 0.25) (layer "F.Cu") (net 39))
 (segment (start 151.13 79.375) (end 151.13 83.377766) (width 0.25) (layer "F.Cu") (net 40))
 (segment (start 153.67 78.74) (end 151.765 78.74) (width 0.25) (layer "F.Cu") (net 40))
 (segment (start 151.13 83.377766) (end 148.577215 85.930551) (width 0.25) (layer "F.Cu") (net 40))
 (segment (start 151.765 78.74) (end 151.13 79.375) (width 0.25) (layer "F.Cu") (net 40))
 (segment (start 150.495 83.30566) (end 148.223662 85.576998) (width 0.25) (layer "F.Cu") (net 41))
 (segment (start 151.13 76.2) (end 150.495 76.835) (width 0.25) (layer "F.Cu") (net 41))
 (segment (start 153.67 76.2) (end 151.13 76.2) (width 0.25) (layer "F.Cu") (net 41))
 (segment (start 150.495 76.835) (end 150.495 83.30566) (width 0.25) (layer "F.Cu") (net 41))
 (segment (start 149.86 83.198198) (end 147.870109 85.188089) (width 0.25) (layer "F.Cu") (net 42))
 (segment (start 147.870109 85.188089) (end 147.870109 85.223445) (width 0.25) (layer "F.Cu") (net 42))
 (segment (start 153.67 73.66) (end 150.495 73.66) (width 0.25) (layer "F.Cu") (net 42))
 (segment (start 150.495 73.66) (end 149.86 74.295) (width 0.25) (layer "F.Cu") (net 42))
 (segment (start 149.86 74.295) (end 149.86 83.198198) (width 0.25) (layer "F.Cu") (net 42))
 (segment (start 149.225 71.755) (end 149.225 83.161446) (width 0.25) (layer "F.Cu") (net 43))
 (segment (start 149.86 71.12) (end 149.225 71.755) (width 0.25) (layer "F.Cu") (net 43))
 (segment (start 149.225 83.161446) (end 147.516555 84.869891) (width 0.25) (layer "F.Cu") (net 43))
 (segment (start 153.67 71.12) (end 149.86 71.12) (width 0.25) (layer "F.Cu") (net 43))
 (segment (start 148.59 83.08934) (end 147.163002 84.516338) (width 0.25) (layer "F.Cu") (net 44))
 (segment (start 148.59 69.215) (end 148.59 83.08934) (width 0.25) (layer "F.Cu") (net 44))
 (segment (start 149.225 68.58) (end 148.59 69.215) (width 0.25) (layer "F.Cu") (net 44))
 (segment (start 153.67 68.58) (end 149.225 68.58) (width 0.25) (layer "F.Cu") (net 44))
 (segment (start 147.955 66.675) (end 147.955 83.017234) (width 0.25) (layer "F.Cu") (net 45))
 (segment (start 147.955 83.017234) (end 146.809449 84.162785) (width 0.25) (layer "F.Cu") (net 45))
 (segment (start 148.59 66.04) (end 147.955 66.675) (width 0.25) (layer "F.Cu") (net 45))
 (segment (start 153.67 66.04) (end 148.59 66.04) (width 0.25) (layer "F.Cu") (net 45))
 (segment (start 147.32 64.135) (end 147.32 82.945126) (width 0.25) (layer "F.Cu") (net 46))
 (segment (start 153.67 63.5) (end 147.955 63.5) (width 0.25) (layer "F.Cu") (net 46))
 (segment (start 147.955 63.5) (end 147.32 64.135) (width 0.25) (layer "F.Cu") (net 46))
 (segment (start 147.32 82.945126) (end 146.455895 83.809231) (width 0.25) (layer "F.Cu") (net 46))
 (segment (start 146.685 82.87302) (end 146.102342 83.455678) (width 0.25) (layer "F.Cu") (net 47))
 (segment (start 147.32 60.96) (end 146.685 61.595) (width 0.25) (layer "F.Cu") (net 47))
 (segment (start 146.685 61.595) (end 146.685 82.87302) (width 0.25) (layer "F.Cu") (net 47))
 (segment (start 153.67 60.96) (end 147.32 60.96) (width 0.25) (layer "F.Cu") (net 47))
 (segment (start 146.05 59.055) (end 146.05 82.800912) (width 0.25) (layer "F.Cu") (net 48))
 (segment (start 146.05 82.800912) (end 145.748788 83.102124) (width 0.25) (layer "F.Cu") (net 48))
 (segment (start 146.685 58.42) (end 146.05 59.055) (width 0.25) (layer "F.Cu") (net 48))
 (segment (start 153.67 58.42) (end 146.685 58.42) (width 0.25) (layer "F.Cu") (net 48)))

